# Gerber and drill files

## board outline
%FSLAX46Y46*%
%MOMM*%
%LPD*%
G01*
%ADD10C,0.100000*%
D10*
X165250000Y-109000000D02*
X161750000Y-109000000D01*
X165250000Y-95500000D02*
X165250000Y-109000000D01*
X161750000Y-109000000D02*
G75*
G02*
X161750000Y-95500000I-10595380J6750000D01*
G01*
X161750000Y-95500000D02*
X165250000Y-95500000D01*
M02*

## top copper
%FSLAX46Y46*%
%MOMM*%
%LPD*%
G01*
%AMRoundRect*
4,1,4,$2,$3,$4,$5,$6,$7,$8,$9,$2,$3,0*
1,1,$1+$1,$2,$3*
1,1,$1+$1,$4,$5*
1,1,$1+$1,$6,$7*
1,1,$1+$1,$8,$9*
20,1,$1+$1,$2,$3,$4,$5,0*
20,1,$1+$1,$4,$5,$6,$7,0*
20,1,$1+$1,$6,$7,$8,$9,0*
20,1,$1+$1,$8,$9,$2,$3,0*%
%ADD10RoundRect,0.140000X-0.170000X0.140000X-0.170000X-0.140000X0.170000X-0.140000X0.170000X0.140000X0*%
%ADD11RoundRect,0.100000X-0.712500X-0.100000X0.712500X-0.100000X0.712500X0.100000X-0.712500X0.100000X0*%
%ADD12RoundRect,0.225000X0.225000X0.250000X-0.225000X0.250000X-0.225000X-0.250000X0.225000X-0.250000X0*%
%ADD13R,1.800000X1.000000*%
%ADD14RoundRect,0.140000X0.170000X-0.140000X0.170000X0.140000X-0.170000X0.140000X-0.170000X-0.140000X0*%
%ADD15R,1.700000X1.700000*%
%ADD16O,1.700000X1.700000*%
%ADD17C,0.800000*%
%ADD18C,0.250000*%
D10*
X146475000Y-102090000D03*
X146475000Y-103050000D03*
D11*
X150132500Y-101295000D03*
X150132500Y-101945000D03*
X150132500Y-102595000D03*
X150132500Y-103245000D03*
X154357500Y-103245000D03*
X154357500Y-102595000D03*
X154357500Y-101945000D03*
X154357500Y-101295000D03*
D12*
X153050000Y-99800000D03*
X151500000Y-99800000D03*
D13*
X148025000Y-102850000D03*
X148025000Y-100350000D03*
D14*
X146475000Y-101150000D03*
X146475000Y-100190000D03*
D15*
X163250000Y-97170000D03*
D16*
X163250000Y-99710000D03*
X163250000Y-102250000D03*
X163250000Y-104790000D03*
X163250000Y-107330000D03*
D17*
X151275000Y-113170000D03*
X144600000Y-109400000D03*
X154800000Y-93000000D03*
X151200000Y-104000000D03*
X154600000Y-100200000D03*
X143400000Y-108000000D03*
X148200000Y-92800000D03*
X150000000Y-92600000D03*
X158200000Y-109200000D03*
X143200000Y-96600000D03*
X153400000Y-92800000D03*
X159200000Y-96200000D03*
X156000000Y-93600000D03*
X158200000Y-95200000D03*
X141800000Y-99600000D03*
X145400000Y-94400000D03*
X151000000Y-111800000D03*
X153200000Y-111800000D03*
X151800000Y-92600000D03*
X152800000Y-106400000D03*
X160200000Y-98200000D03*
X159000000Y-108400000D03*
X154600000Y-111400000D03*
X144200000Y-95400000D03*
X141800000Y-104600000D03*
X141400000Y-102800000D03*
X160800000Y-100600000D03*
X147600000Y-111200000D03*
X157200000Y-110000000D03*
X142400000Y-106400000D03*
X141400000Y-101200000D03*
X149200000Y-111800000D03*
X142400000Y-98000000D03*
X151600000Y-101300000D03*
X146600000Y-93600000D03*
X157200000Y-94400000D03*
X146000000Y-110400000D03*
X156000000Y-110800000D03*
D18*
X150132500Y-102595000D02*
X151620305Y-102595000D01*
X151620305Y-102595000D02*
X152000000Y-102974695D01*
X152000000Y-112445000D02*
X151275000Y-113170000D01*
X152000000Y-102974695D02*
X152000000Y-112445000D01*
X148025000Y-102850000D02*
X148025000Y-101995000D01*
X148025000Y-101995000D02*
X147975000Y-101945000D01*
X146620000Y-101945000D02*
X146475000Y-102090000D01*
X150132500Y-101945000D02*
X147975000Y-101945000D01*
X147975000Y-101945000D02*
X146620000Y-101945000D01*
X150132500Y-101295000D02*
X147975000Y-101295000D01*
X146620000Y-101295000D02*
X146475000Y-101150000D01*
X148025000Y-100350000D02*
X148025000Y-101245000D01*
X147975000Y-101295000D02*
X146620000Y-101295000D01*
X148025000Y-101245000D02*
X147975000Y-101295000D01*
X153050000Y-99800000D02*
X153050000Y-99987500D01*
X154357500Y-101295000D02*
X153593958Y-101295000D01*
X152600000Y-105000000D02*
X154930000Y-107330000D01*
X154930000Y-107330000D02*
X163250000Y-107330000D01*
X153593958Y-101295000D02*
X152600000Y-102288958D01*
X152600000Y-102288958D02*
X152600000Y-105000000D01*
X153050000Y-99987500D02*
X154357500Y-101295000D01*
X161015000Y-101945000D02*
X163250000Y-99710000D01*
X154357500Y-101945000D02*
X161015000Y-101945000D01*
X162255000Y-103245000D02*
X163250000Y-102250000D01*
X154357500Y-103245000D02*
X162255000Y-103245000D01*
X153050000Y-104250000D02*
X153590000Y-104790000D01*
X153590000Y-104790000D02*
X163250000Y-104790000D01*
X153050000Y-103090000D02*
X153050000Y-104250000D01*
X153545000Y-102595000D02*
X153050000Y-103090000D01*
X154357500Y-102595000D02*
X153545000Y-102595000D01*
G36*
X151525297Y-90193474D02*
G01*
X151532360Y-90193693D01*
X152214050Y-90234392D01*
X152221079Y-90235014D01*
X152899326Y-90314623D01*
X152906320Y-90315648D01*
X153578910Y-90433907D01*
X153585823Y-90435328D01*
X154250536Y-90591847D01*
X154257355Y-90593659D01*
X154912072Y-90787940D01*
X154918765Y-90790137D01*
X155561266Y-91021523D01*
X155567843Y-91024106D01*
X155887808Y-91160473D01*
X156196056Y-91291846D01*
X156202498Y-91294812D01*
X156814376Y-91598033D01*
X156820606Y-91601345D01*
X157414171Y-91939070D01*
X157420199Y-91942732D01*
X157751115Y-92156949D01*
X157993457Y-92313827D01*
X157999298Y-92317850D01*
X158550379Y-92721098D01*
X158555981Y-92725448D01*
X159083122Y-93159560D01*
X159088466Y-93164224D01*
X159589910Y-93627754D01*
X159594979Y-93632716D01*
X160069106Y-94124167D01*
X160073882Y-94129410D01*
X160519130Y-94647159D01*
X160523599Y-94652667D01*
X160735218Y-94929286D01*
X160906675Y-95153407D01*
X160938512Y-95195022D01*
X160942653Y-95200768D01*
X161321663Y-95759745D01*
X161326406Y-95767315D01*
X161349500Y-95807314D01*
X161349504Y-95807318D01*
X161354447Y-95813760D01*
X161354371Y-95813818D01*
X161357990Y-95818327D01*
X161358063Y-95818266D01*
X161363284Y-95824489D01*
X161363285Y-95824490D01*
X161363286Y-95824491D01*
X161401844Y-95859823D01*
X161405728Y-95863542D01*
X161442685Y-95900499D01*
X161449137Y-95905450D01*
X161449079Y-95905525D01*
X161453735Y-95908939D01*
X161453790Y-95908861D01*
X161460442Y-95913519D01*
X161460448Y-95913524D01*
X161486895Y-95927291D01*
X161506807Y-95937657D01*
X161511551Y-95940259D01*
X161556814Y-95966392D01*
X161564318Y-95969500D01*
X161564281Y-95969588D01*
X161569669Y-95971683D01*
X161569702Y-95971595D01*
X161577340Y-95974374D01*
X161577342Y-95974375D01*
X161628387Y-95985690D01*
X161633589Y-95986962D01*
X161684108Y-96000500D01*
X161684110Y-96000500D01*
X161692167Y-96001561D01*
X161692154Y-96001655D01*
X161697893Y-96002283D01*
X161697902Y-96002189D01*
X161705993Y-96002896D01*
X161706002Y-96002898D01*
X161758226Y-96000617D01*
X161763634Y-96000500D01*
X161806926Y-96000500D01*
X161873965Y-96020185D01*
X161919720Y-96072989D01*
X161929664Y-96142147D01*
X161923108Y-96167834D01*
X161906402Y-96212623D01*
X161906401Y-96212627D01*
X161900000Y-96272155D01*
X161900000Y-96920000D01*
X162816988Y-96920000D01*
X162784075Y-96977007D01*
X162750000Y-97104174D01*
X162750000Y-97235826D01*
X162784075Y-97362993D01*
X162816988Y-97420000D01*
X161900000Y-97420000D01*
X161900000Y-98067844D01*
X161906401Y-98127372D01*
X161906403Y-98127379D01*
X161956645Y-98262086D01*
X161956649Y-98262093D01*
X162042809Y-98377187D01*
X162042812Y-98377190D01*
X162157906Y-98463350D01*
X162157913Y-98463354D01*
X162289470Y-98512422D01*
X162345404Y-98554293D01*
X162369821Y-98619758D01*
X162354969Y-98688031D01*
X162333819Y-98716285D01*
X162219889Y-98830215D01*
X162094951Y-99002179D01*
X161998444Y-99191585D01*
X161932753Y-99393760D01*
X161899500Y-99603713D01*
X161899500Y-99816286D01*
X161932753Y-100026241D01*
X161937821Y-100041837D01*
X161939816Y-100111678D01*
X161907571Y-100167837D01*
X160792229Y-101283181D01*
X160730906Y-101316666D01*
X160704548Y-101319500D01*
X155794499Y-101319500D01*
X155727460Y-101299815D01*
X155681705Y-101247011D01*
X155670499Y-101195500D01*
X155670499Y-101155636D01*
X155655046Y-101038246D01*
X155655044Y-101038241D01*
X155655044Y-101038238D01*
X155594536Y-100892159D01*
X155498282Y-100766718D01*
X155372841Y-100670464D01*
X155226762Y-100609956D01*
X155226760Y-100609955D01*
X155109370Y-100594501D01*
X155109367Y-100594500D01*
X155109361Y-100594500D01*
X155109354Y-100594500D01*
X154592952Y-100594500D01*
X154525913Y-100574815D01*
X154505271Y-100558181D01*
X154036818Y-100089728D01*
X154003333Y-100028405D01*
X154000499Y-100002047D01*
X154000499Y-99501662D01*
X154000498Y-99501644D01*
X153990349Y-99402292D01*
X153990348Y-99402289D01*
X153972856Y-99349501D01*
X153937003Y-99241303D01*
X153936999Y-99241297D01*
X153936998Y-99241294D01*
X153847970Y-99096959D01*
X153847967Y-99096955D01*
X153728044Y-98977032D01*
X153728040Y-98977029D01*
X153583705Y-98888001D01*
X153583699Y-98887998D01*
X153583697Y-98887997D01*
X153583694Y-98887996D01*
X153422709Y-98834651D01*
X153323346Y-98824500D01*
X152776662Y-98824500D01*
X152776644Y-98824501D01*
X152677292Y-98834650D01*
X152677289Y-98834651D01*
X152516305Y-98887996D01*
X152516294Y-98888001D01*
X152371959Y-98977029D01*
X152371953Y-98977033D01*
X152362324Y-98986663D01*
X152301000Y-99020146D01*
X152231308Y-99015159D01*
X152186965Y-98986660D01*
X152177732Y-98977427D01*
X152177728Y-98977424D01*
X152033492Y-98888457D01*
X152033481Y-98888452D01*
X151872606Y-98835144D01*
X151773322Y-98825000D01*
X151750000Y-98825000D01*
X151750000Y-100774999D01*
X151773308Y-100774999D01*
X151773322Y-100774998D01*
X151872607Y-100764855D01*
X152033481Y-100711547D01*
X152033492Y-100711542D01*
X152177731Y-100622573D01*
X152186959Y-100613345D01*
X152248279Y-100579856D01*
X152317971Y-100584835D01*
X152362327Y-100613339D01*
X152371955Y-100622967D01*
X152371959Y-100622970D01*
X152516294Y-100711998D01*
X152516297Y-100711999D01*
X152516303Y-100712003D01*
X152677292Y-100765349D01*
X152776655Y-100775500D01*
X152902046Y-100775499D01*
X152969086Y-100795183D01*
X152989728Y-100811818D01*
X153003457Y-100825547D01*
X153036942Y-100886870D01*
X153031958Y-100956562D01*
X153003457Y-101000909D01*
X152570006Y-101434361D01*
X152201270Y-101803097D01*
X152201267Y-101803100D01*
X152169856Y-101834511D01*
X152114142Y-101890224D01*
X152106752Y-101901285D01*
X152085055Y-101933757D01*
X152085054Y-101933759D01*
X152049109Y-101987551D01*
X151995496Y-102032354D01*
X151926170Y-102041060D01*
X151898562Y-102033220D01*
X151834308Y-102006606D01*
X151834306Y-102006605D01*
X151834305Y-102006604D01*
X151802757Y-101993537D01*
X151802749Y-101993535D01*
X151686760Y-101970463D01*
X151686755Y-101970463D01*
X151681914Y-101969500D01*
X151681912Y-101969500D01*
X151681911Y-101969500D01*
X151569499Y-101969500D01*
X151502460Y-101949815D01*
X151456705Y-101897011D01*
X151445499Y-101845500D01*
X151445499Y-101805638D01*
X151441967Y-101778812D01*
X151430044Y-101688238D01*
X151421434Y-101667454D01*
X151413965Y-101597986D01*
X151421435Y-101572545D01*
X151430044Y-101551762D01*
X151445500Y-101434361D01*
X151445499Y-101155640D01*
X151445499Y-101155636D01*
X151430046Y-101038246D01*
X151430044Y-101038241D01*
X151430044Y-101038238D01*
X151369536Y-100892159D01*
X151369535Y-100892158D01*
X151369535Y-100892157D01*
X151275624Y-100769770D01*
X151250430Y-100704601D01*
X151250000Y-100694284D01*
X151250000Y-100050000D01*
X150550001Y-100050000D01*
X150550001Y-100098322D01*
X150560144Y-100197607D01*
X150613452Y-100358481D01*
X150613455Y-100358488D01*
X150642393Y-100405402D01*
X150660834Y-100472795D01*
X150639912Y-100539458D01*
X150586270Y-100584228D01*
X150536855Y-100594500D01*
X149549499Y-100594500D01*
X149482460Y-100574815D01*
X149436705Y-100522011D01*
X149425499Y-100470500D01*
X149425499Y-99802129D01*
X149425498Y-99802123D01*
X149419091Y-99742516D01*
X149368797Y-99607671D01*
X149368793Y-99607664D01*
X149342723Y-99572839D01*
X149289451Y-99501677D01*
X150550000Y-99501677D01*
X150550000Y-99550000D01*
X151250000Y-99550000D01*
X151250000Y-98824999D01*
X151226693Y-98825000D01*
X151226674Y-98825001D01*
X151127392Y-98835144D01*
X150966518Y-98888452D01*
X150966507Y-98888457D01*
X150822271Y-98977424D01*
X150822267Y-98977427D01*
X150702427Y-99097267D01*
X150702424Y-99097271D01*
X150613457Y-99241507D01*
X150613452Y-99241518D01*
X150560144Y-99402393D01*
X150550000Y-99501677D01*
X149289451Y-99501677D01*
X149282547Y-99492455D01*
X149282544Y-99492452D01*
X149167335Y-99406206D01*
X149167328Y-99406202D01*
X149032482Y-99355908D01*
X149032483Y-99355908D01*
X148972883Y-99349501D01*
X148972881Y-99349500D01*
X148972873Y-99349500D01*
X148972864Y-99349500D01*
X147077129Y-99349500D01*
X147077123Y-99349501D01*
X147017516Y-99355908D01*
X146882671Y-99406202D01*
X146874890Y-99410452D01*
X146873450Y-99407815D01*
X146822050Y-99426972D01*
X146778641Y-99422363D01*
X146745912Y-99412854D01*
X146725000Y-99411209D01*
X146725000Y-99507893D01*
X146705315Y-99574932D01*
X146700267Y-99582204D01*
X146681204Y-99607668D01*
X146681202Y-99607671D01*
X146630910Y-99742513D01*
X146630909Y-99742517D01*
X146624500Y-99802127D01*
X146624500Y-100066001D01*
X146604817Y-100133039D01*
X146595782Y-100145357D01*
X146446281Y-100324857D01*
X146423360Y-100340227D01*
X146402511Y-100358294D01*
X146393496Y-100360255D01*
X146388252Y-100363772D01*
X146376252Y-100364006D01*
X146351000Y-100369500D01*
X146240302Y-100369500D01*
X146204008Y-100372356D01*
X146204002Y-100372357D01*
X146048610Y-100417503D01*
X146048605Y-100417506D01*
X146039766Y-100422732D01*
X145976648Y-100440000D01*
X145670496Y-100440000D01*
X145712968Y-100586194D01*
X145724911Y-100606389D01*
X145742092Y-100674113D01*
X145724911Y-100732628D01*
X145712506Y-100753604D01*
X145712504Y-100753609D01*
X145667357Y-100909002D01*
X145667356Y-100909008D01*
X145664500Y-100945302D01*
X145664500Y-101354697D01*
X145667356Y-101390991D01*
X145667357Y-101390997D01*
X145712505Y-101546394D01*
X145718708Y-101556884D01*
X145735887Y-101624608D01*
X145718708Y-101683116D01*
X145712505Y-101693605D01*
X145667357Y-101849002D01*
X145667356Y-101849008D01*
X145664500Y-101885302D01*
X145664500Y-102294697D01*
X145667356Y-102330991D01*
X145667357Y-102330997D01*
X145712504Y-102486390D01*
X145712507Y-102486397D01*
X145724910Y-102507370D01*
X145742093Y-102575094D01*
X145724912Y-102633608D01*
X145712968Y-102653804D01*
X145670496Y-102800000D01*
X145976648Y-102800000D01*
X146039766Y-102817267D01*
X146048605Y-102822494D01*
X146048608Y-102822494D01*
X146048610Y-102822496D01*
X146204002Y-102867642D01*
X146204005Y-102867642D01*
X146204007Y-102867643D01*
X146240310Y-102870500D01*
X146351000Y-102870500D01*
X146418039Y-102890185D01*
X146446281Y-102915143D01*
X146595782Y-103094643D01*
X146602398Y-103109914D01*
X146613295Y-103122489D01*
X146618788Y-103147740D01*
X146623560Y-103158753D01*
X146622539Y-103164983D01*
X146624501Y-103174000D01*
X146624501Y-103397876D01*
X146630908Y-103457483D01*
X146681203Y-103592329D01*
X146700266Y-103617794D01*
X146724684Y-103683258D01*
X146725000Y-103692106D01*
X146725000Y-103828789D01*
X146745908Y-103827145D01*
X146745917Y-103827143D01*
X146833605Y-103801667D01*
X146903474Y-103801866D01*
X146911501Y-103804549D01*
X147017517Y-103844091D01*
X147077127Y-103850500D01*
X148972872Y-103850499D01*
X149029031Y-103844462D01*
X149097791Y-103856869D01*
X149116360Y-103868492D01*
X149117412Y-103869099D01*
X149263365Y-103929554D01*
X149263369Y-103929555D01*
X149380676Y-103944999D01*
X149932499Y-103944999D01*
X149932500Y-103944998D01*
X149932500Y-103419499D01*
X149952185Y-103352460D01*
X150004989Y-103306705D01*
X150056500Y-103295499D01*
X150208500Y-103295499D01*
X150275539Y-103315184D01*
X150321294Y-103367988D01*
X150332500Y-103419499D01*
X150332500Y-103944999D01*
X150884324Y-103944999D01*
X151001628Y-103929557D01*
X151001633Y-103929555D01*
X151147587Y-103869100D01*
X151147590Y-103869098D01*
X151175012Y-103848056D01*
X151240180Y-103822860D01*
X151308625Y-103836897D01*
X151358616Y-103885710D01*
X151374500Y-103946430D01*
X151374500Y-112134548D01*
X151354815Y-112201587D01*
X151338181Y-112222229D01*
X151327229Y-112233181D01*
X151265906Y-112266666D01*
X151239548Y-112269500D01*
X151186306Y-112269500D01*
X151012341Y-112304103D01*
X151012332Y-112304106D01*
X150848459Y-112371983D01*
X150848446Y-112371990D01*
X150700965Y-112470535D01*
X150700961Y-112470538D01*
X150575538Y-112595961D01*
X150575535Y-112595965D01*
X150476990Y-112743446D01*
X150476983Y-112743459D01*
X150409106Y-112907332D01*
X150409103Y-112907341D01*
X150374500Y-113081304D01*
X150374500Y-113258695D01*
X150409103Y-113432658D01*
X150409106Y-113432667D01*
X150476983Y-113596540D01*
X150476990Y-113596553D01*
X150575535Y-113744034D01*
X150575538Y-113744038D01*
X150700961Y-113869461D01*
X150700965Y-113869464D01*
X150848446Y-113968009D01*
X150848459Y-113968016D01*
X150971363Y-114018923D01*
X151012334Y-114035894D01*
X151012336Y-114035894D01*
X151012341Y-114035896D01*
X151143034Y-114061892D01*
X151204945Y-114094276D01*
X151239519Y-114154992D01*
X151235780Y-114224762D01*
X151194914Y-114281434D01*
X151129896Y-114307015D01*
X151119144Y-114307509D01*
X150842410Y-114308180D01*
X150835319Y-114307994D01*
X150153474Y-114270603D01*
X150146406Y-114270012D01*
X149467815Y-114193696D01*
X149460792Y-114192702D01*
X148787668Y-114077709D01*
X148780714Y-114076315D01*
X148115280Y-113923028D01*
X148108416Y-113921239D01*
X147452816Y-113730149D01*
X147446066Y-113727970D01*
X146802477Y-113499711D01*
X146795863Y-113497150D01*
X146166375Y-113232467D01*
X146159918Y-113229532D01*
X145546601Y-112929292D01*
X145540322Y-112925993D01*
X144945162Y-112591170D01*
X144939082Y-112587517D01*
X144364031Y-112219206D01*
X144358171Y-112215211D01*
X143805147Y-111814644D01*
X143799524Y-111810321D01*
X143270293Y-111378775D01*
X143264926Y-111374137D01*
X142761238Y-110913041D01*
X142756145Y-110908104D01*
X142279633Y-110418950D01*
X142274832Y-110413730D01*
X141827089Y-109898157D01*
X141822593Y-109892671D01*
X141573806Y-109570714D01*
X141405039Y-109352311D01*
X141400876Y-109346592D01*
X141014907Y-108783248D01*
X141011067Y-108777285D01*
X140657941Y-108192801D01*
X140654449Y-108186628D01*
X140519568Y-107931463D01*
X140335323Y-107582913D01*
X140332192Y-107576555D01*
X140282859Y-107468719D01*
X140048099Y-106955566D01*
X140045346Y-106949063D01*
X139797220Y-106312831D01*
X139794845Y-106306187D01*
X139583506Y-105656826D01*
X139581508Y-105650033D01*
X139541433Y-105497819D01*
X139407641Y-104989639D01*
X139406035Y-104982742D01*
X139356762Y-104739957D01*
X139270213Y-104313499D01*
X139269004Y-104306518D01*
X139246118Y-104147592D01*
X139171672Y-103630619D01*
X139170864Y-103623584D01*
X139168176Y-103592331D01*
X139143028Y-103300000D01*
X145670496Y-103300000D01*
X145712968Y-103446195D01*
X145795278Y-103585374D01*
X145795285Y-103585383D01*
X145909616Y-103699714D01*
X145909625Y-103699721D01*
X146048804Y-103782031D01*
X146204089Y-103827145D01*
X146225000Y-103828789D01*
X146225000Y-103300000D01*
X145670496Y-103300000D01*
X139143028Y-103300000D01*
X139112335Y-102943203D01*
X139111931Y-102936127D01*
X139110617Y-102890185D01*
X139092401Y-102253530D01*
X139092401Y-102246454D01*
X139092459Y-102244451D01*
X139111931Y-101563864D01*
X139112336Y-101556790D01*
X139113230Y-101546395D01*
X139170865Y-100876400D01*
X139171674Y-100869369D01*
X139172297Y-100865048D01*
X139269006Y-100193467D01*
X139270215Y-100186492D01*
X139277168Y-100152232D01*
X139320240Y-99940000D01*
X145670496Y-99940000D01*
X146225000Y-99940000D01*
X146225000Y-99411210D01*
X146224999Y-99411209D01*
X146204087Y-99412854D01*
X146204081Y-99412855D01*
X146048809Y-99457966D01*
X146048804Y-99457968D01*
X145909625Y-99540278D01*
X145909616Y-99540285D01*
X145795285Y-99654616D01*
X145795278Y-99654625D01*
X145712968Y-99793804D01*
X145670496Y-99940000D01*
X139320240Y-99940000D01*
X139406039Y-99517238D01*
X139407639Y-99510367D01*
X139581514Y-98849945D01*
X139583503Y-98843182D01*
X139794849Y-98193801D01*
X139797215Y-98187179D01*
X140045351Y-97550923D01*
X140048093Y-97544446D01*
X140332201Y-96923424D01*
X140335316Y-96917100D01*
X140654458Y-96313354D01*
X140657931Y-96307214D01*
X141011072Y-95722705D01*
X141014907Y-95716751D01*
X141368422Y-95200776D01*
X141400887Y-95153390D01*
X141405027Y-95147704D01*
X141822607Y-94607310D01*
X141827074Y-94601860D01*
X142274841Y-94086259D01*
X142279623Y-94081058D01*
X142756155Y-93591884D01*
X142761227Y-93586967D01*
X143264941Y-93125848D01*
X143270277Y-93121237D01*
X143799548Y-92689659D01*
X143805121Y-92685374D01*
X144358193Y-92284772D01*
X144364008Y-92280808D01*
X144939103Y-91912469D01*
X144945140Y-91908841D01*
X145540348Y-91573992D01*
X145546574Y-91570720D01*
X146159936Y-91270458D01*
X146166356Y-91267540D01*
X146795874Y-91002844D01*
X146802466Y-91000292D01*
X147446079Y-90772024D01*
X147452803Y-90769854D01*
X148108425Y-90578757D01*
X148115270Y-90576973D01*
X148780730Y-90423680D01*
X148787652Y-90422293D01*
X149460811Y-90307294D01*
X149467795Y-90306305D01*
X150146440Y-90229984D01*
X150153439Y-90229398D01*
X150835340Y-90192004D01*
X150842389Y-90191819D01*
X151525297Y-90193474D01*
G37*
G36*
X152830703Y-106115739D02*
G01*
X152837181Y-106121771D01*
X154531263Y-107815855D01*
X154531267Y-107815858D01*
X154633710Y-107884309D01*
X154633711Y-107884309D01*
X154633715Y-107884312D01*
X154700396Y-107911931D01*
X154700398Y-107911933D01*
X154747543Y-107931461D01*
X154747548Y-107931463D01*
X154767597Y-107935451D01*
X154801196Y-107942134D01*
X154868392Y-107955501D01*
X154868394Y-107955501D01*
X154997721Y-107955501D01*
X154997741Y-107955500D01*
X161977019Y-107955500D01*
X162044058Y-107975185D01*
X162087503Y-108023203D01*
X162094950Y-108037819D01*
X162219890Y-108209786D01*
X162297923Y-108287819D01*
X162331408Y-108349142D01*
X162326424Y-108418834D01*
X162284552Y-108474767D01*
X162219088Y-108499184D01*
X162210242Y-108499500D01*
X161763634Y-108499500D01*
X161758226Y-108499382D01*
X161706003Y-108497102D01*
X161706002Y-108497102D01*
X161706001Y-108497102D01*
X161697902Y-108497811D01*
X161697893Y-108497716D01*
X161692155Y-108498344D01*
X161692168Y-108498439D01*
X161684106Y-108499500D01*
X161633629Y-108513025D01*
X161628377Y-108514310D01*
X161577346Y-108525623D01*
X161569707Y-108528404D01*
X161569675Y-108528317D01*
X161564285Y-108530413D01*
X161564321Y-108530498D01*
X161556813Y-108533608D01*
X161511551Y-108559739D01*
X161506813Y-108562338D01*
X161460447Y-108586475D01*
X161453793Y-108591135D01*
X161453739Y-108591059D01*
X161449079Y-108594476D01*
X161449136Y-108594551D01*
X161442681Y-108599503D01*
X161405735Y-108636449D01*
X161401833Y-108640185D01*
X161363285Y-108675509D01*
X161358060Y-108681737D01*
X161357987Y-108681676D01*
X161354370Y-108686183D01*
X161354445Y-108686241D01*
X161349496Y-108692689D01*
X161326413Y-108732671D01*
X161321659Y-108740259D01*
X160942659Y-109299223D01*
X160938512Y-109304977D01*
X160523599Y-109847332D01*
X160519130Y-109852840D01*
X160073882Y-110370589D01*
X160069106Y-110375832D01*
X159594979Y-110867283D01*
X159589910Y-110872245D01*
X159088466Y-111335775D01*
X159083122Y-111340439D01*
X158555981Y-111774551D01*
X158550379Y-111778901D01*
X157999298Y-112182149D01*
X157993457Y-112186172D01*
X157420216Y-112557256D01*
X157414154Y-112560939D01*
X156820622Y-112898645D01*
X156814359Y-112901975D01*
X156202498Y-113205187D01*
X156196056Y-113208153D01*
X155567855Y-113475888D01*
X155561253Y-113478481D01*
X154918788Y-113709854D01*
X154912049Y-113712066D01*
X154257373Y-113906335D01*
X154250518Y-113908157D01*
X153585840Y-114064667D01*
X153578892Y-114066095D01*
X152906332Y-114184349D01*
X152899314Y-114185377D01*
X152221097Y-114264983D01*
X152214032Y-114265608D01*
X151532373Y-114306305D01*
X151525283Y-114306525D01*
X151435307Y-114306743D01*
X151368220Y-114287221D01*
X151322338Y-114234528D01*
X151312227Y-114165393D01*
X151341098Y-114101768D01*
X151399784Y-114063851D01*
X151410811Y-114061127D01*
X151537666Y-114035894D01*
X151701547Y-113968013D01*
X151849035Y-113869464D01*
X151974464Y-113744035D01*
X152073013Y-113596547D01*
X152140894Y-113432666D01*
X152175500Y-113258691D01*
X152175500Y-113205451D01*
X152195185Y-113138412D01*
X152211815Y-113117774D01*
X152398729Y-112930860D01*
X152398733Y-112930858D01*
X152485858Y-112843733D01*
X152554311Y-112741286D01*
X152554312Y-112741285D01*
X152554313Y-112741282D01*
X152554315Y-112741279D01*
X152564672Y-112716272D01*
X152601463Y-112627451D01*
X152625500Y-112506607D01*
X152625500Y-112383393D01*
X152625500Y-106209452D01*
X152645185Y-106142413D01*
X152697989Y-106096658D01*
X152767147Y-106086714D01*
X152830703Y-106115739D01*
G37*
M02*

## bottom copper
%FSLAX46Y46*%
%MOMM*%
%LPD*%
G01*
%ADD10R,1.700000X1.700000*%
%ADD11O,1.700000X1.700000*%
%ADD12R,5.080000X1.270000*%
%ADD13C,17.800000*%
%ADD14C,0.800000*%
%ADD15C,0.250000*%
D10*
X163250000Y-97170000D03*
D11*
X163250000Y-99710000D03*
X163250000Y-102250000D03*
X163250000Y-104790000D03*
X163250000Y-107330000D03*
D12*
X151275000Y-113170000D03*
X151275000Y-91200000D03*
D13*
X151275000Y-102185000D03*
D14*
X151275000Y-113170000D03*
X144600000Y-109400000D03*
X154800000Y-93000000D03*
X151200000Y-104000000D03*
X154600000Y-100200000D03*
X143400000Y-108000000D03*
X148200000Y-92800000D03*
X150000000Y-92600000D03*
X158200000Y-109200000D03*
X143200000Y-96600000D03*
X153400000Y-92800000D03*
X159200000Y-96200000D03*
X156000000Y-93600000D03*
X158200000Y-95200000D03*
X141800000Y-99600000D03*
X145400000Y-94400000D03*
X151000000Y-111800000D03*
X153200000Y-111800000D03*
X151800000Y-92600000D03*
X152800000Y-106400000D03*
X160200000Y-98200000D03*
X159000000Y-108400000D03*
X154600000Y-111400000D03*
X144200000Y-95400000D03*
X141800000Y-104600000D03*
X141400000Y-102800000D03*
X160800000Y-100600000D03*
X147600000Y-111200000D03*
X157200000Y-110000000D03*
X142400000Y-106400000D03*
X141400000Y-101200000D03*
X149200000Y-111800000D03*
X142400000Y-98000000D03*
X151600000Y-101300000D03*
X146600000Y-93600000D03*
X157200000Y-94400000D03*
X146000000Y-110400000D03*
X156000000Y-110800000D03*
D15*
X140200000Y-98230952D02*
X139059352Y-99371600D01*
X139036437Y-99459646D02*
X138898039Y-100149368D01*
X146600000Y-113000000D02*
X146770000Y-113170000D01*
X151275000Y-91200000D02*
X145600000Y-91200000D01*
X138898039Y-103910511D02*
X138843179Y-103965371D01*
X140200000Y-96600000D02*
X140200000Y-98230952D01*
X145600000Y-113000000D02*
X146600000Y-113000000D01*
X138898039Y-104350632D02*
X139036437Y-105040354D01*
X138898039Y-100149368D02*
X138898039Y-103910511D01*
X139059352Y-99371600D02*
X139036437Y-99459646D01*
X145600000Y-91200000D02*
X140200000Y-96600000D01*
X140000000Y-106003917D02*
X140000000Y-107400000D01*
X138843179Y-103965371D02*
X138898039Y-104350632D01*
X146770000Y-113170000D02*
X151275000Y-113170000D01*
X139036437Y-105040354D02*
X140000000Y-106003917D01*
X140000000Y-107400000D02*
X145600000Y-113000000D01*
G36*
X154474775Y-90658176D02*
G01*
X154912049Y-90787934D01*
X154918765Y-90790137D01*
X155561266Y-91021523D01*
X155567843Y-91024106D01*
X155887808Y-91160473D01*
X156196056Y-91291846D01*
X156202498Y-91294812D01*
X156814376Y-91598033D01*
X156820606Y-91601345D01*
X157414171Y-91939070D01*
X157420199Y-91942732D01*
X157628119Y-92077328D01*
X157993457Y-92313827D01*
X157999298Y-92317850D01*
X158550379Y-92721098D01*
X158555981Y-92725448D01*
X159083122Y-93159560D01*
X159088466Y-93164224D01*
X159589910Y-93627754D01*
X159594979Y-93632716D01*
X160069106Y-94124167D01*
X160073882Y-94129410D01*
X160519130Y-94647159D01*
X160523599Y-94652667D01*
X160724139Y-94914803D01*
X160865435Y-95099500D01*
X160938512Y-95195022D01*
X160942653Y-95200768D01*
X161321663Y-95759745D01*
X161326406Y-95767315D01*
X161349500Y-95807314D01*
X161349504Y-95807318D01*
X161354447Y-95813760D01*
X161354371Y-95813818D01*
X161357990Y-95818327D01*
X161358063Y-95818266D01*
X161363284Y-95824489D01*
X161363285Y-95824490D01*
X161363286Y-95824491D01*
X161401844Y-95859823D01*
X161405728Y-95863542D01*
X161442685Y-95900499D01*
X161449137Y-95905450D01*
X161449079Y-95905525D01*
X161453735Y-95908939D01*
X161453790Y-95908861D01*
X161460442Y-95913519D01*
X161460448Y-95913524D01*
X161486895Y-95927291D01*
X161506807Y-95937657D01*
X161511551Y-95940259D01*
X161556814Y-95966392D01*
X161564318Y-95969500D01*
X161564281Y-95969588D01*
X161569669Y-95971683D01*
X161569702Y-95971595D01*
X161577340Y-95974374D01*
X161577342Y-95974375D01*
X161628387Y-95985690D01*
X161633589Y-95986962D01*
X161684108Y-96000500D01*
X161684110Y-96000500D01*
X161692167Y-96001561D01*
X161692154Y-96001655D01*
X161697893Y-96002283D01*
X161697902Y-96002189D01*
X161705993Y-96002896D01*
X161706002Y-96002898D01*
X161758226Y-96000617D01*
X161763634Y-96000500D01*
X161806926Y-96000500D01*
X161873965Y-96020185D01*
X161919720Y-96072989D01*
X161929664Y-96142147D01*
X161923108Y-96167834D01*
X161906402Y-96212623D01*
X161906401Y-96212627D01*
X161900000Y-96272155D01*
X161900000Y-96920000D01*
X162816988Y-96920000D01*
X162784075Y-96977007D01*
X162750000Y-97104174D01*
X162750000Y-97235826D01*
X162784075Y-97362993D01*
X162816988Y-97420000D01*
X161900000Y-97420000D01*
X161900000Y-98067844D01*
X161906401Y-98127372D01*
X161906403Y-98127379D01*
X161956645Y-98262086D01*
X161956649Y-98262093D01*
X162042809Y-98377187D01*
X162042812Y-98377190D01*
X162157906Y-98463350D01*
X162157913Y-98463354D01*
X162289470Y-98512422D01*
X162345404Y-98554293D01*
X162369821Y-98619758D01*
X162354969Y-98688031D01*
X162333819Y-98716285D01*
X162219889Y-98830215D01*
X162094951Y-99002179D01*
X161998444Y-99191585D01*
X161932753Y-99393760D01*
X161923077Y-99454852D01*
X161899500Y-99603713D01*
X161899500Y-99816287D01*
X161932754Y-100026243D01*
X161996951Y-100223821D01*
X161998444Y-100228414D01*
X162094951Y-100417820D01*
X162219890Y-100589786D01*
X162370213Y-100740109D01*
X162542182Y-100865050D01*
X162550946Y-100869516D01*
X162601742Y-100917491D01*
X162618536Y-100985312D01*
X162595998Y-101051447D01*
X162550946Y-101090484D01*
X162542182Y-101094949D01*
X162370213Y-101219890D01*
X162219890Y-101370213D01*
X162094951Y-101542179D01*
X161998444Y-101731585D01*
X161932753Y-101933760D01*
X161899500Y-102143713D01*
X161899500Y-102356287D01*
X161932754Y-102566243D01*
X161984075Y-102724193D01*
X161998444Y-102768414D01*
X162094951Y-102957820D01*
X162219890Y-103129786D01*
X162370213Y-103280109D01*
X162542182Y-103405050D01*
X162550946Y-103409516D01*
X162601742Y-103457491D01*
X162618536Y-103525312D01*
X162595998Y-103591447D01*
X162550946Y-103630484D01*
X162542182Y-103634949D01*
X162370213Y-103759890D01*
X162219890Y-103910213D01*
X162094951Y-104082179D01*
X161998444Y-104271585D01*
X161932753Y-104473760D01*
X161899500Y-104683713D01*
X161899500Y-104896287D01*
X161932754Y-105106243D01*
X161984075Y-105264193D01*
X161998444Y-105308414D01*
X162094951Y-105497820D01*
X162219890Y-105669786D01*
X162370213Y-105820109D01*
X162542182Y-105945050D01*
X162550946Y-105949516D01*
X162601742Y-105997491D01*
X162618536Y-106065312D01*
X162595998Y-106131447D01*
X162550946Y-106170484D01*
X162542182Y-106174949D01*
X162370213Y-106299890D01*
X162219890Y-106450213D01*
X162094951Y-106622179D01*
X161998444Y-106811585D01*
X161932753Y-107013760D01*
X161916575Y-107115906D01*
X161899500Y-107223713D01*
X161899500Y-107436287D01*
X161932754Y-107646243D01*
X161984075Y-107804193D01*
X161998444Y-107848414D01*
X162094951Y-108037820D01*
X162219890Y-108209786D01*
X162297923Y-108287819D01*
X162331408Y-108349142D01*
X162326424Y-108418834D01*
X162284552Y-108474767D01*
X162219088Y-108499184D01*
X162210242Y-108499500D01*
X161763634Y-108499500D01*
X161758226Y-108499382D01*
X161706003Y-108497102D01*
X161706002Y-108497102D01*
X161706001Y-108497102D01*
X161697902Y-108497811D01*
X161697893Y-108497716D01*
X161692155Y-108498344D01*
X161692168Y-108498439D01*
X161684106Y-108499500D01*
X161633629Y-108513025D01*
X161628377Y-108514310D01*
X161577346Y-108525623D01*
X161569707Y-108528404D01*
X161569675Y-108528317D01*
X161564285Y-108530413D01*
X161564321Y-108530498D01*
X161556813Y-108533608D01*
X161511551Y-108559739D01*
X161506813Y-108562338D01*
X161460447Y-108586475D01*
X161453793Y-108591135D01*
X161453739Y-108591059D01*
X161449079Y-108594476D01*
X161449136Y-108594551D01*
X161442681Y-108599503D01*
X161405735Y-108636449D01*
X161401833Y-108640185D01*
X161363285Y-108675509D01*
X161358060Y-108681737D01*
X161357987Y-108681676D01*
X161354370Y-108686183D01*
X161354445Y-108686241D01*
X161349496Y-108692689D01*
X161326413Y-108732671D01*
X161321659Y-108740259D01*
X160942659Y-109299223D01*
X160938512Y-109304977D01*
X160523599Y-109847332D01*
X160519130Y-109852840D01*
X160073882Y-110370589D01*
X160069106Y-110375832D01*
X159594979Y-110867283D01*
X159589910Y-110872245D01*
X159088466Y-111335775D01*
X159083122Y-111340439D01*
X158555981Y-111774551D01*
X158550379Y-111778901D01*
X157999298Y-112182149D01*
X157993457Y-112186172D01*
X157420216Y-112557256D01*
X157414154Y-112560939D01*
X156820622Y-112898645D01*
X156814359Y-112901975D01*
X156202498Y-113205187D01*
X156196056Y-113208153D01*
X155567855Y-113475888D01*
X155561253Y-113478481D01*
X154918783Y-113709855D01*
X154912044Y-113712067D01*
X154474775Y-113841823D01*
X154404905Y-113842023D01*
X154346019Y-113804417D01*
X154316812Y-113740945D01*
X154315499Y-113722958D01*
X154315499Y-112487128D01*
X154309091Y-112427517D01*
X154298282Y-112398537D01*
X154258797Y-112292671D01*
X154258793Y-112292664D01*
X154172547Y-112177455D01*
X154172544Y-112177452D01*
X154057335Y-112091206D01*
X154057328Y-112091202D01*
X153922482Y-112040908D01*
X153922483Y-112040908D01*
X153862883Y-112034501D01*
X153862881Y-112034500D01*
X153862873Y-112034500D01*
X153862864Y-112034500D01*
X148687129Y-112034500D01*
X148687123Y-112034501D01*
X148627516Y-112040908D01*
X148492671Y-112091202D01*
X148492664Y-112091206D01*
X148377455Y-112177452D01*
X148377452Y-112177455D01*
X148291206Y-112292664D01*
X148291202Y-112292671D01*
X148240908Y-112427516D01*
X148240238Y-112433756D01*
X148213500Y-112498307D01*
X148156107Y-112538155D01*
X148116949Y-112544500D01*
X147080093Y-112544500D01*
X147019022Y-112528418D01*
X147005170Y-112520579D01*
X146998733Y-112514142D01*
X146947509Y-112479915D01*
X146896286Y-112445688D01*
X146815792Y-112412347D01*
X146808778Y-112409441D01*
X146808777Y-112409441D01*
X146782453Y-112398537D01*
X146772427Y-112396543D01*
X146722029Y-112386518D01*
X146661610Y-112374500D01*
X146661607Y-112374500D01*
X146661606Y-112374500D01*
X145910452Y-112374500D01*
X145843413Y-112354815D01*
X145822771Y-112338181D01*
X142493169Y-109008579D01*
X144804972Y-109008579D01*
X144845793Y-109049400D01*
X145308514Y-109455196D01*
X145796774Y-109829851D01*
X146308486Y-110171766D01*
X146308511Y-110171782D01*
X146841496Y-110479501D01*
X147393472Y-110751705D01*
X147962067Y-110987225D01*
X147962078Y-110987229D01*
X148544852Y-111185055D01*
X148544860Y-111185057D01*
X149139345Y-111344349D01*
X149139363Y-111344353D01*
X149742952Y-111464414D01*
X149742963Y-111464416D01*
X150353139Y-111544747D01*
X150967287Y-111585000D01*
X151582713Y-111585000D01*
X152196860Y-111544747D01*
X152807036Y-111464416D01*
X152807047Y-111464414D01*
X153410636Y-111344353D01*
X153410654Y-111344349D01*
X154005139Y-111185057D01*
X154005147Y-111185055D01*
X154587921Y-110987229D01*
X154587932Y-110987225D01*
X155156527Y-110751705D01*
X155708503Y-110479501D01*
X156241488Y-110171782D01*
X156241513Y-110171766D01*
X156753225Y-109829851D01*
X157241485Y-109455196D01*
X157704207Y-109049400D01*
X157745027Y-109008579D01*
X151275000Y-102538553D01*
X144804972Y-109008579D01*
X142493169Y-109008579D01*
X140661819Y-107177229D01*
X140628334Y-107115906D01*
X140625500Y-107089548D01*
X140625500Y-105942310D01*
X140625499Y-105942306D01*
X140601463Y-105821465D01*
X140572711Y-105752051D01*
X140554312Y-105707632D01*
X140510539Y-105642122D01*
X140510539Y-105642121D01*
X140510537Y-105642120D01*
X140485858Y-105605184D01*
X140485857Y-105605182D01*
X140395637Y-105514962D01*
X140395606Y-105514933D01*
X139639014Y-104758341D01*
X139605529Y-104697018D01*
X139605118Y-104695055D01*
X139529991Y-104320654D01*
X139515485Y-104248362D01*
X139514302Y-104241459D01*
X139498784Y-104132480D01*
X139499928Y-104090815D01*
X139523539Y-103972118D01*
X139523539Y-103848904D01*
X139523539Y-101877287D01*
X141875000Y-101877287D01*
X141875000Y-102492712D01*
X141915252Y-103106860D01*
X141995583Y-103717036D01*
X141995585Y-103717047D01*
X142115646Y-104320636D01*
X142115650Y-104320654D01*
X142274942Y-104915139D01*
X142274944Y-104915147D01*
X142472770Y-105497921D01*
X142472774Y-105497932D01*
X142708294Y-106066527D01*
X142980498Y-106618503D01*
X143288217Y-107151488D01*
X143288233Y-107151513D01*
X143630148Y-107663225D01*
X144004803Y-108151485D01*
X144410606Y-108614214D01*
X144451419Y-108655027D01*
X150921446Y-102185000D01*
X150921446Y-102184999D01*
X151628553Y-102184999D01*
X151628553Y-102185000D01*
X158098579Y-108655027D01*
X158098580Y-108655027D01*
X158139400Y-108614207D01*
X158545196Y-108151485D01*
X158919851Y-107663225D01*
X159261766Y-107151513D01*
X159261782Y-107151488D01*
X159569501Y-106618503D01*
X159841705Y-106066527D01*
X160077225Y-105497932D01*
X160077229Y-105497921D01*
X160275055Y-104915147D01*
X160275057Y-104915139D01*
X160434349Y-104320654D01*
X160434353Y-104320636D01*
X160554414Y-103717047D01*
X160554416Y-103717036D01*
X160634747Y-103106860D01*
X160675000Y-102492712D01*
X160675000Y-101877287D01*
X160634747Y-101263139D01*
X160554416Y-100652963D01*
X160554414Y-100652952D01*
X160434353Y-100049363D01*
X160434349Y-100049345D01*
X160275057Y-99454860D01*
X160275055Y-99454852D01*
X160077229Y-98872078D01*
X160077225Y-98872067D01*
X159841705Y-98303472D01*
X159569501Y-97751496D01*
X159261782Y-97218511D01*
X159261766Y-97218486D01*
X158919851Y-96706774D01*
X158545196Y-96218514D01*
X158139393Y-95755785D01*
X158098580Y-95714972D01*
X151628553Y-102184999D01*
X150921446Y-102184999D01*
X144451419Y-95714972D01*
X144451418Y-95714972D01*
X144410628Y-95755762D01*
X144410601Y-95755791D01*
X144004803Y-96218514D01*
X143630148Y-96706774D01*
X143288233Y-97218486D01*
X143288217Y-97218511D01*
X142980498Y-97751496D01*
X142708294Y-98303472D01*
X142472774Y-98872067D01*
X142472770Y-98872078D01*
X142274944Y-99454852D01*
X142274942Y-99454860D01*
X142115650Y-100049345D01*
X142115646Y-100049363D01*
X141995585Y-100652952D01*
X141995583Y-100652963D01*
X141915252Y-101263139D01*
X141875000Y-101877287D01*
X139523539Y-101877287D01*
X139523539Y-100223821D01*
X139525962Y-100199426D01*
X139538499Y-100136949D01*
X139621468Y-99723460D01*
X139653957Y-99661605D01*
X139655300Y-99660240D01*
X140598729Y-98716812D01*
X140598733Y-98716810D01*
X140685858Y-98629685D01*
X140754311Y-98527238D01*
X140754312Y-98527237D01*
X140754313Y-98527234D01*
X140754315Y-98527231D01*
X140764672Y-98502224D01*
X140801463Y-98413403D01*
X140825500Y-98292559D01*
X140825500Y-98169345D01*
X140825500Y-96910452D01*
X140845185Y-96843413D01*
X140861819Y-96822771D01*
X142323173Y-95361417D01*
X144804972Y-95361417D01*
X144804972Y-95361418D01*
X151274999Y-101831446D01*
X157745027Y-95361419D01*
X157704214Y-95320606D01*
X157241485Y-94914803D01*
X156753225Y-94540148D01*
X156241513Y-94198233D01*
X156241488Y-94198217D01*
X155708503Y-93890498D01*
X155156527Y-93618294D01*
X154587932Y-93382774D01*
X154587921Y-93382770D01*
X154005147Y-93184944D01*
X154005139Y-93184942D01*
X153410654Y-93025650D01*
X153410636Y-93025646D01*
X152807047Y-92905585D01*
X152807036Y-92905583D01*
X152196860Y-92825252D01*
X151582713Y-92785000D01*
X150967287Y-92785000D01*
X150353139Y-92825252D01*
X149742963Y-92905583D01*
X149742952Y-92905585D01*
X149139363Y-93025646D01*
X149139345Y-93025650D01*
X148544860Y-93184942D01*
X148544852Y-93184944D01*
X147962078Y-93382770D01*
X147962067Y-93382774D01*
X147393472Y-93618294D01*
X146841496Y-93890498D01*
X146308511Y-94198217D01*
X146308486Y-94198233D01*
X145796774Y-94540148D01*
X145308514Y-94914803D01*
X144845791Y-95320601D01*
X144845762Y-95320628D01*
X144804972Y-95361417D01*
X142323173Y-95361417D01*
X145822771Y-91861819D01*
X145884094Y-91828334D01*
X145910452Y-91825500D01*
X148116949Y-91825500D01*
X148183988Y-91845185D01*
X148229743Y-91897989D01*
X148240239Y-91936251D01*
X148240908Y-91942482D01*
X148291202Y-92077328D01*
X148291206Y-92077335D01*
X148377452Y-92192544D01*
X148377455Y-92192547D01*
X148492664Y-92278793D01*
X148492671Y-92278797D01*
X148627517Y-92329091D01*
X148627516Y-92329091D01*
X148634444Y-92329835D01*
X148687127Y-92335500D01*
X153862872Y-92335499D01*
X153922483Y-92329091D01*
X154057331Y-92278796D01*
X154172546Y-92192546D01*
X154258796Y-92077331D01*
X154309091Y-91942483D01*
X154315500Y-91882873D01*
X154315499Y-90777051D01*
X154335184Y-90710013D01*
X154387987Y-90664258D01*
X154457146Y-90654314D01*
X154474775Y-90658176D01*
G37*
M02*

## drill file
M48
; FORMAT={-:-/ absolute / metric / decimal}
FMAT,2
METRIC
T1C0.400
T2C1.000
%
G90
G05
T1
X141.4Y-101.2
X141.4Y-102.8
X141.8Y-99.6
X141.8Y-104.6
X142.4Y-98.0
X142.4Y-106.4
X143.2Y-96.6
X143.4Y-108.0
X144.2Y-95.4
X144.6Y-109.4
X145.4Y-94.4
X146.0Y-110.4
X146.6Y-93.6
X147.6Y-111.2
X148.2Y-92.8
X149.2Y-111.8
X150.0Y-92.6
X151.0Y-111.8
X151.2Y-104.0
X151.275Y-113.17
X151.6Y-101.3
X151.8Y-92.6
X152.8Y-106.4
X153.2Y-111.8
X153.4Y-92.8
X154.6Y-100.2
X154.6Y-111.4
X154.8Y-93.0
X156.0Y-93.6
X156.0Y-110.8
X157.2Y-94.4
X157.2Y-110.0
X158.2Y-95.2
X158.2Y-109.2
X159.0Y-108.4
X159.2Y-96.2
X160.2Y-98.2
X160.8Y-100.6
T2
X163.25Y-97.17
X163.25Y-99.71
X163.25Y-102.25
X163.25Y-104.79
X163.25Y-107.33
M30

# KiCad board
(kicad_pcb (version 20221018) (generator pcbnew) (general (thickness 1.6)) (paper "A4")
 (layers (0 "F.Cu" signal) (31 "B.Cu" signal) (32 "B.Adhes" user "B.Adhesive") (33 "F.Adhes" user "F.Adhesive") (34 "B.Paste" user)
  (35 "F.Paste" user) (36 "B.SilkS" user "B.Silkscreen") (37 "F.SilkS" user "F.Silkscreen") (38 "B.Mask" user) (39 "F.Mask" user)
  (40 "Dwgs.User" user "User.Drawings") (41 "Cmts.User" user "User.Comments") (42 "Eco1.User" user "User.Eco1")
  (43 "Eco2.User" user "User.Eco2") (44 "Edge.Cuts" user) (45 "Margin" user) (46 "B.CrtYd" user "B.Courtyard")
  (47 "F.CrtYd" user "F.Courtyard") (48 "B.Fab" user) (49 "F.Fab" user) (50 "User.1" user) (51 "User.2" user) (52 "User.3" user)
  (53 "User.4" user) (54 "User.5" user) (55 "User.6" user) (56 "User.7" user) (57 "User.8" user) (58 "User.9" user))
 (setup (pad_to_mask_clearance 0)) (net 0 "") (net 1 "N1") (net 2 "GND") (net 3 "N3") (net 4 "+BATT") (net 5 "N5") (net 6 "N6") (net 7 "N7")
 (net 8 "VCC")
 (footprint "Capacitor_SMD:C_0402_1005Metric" (layer "F.Cu") (at 146.475 102.57 -90)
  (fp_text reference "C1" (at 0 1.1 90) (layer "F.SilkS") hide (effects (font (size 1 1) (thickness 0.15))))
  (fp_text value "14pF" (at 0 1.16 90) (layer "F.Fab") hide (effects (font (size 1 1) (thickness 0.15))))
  (pad "1" smd roundrect (at -0.48 0 270) (size 0.56 0.62) (layers "F.Cu" "F.Paste" "F.Mask") (roundrect_rratio 0.25) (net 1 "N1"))
  (pad "2" smd roundrect (at 0.48 0 270) (size 0.56 0.62) (layers "F.Cu" "F.Paste" "F.Mask") (roundrect_rratio 0.25) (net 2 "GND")))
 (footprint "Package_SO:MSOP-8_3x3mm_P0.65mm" (layer "F.Cu") (at 152.245 102.27)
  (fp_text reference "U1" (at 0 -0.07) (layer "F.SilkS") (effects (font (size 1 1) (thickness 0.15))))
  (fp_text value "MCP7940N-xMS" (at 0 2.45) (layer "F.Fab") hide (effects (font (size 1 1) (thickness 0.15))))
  (pad "1" smd roundrect (at -2.1125 -0.975) (size 1.625 0.4) (layers "F.Cu" "F.Paste" "F.Mask") (roundrect_rratio 0.25) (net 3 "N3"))
  (pad "2" smd roundrect (at -2.1125 -0.325) (size 1.625 0.4) (layers "F.Cu" "F.Paste" "F.Mask") (roundrect_rratio 0.25) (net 1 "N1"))
  (pad "3" smd roundrect (at -2.1125 0.325) (size 1.625 0.4) (layers "F.Cu" "F.Paste" "F.Mask") (roundrect_rratio 0.25) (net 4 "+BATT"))
  (pad "4" smd roundrect (at -2.1125 0.975) (size 1.625 0.4) (layers "F.Cu" "F.Paste" "F.Mask") (roundrect_rratio 0.25) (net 2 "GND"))
  (pad "5" smd roundrect (at 2.1125 0.975) (size 1.625 0.4) (layers "F.Cu" "F.Paste" "F.Mask") (roundrect_rratio 0.25) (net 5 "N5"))
  (pad "6" smd roundrect (at 2.1125 0.325) (size 1.625 0.4) (layers "F.Cu" "F.Paste" "F.Mask") (roundrect_rratio 0.25) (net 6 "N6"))
  (pad "7" smd roundrect (at 2.1125 -0.325) (size 1.625 0.4) (layers "F.Cu" "F.Paste" "F.Mask") (roundrect_rratio 0.25) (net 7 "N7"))
  (pad "8" smd roundrect (at 2.1125 -0.975) (size 1.625 0.4) (layers "F.Cu" "F.Paste" "F.Mask") (roundrect_rratio 0.25) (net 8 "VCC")))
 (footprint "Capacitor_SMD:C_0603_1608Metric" (layer "F.Cu") (at 152.275 99.8 180)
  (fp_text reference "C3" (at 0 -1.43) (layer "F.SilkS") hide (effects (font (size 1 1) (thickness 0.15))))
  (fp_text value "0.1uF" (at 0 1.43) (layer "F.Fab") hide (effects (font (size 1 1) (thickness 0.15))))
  (pad "1" smd roundrect (at -0.775 0 180) (size 0.9 0.95) (layers "F.Cu" "F.Paste" "F.Mask") (roundrect_rratio 0.25) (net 8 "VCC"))
  (pad "2" smd roundrect (at 0.775 0 180) (size 0.9 0.95) (layers "F.Cu" "F.Paste" "F.Mask") (roundrect_rratio 0.25) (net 2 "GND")))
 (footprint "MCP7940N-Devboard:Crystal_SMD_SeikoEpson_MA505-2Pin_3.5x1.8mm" (layer "F.Cu") (at 148.025 101.6 90)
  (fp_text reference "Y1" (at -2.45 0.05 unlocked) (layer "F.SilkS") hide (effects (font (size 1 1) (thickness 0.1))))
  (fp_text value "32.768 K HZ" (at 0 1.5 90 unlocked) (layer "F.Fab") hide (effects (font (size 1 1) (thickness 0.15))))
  (pad "1" smd rect (at -1.25 0 90) (size 1 1.8) (layers "F.Cu" "F.Paste" "F.Mask") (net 1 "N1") (thermal_bridge_angle 45))
  (pad "2" smd rect (at 1.25 0 90) (size 1 1.8) (layers "F.Cu" "F.Paste" "F.Mask") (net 3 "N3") (thermal_bridge_angle 45)))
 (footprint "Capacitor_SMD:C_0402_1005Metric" (layer "F.Cu") (at 146.475 100.67 90)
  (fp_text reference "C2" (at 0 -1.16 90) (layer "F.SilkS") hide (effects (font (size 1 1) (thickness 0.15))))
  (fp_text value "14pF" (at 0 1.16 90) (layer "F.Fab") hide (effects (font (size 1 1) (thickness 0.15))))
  (pad "1" smd roundrect (at -0.48 0 90) (size 0.56 0.62) (layers "F.Cu" "F.Paste" "F.Mask") (roundrect_rratio 0.25) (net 3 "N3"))
  (pad "2" smd roundrect (at 0.48 0 90) (size 0.56 0.62) (layers "F.Cu" "F.Paste" "F.Mask") (roundrect_rratio 0.25) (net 2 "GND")))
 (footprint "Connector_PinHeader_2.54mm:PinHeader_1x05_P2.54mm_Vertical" (layer "F.Cu") (at 163.25 97.17)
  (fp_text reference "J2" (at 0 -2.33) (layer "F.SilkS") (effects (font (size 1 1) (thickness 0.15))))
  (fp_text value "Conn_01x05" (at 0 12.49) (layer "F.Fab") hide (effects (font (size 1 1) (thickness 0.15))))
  (pad "1" thru_hole rect (at 0 0) (size 1.7 1.7) (drill 1) (layers "*.Cu" "*.Mask") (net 2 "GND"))
  (pad "2" thru_hole oval (at 0 2.54) (size 1.7 1.7) (drill 1) (layers "*.Cu" "*.Mask") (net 7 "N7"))
  (pad "3" thru_hole oval (at 0 5.08) (size 1.7 1.7) (drill 1) (layers "*.Cu" "*.Mask") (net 5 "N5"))
  (pad "4" thru_hole oval (at 0 7.62) (size 1.7 1.7) (drill 1) (layers "*.Cu" "*.Mask") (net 6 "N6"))
  (pad "5" thru_hole oval (at 0 10.16) (size 1.7 1.7) (drill 1) (layers "*.Cu" "*.Mask") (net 8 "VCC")))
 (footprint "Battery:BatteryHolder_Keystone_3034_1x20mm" (layer "B.Cu") (at 151.275 102.185 90)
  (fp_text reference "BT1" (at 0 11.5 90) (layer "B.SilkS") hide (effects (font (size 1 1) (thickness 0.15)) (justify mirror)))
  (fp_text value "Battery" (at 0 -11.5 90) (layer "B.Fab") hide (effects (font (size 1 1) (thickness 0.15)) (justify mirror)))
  (pad "1" smd rect (at -10.985 0 90) (size 1.27 5.08) (layers "B.Cu" "B.Paste" "B.Mask") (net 4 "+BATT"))
  (pad "1" smd rect (at 10.985 0 90) (size 1.27 5.08) (layers "B.Cu" "B.Paste" "B.Mask") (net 4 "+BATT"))
  (pad "2" smd circle (at 0 0 90) (size 17.8 17.8) (layers "B.Cu" "B.Mask") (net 2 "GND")))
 (gr_line (start 165.25 109) (end 161.75 109) (stroke (width 0.1) (type default)) (layer "Edge.Cuts"))
 (gr_line (start 165.25 95.5) (end 165.25 109) (stroke (width 0.1) (type default)) (layer "Edge.Cuts"))
 (gr_arc (start 161.75 109) (mid 138.5918 102.25) (end 161.75 95.5) (stroke (width 0.1) (type default)) (layer "Edge.Cuts"))
 (gr_line (start 161.75 95.5) (end 165.25 95.5) (stroke (width 0.1) (type default)) (layer "Edge.Cuts"))
 (segment (start 150.1325 102.595) (end 151.620305 102.595) (width 0.25) (layer "F.Cu") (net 4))
 (segment (start 151.620305 102.595) (end 152 102.974695) (width 0.25) (layer "F.Cu") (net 4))
 (segment (start 152 112.445) (end 151.275 113.17) (width 0.25) (layer "F.Cu") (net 4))
 (segment (start 152 102.974695) (end 152 112.445) (width 0.25) (layer "F.Cu") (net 4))
 (via (at 151.275 113.17) (size 0.8) (drill 0.4) (layers "F.Cu" "B.Cu") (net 4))
 (segment (start 140.2 98.230952) (end 139.059352 99.3716) (width 0.25) (layer "B.Cu") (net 4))
 (segment (start 139.036437 99.459646) (end 138.898039 100.149368) (width 0.25) (layer "B.Cu") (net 4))
 (segment (start 146.6 113) (end 146.77 113.17) (width 0.25) (layer "B.Cu") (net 4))
 (segment (start 151.275 91.2) (end 145.6 91.2) (width 0.25) (layer "B.Cu") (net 4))
 (segment (start 138.898039 103.910511) (end 138.843179 103.965371) (width 0.25) (layer "B.Cu") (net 4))
 (segment (start 140.2 96.6) (end 140.2 98.230952) (width 0.25) (layer "B.Cu") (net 4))
 (segment (start 145.6 113) (end 146.6 113) (width 0.25) (layer "B.Cu") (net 4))
 (segment (start 138.898039 104.350632) (end 139.036437 105.040354) (width 0.25) (layer "B.Cu") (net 4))
 (segment (start 138.898039 100.149368) (end 138.898039 103.910511) (width 0.25) (layer "B.Cu") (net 4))
 (segment (start 139.059352 99.3716) (end 139.036437 99.459646) (width 0.25) (layer "B.Cu") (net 4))
 (segment (start 145.6 91.2) (end 140.2 96.6) (width 0.25) (layer "B.Cu") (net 4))
 (segment (start 140 106.003917) (end 140 107.4) (width 0.25) (layer "B.Cu") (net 4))
 (segment (start 138.843179 103.965371) (end 138.898039 104.350632) (width 0.25) (layer "B.Cu") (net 4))
 (segment (start 146.77 113.17) (end 151.275 113.17) (width 0.25) (layer "B.Cu") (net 4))
 (segment (start 139.036437 105.040354) (end 140 106.003917) (width 0.25) (layer "B.Cu") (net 4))
 (segment (start 140 107.4) (end 145.6 113) (width 0.25) (layer "B.Cu") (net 4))
 (via (at 144.6 109.4) (size 0.8) (drill 0.4) (layers "F.Cu" "B.Cu") (free) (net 2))
 (via (at 154.8 93) (size 0.8) (drill 0.4) (layers "F.Cu" "B.Cu") (free) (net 2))
 (via (at 151.2 104) (size 0.8) (drill 0.4) (layers "F.Cu" "B.Cu") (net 2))
 (via (at 154.6 100.2) (size 0.8) (drill 0.4) (layers "F.Cu" "B.Cu") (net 2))
 (via (at 143.4 108) (size 0.8) (drill 0.4) (layers "F.Cu" "B.Cu") (free) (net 2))
 (via (at 148.2 92.8) (size 0.8) (drill 0.4) (layers "F.Cu" "B.Cu") (free) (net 2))
 (via (at 150 92.6) (size 0.8) (drill 0.4) (layers "F.Cu" "B.Cu") (free) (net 2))
 (via (at 158.2 109.2) (size 0.8) (drill 0.4) (layers "F.Cu" "B.Cu") (free) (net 2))
 (via (at 143.2 96.6) (size 0.8) (drill 0.4) (layers "F.Cu" "B.Cu") (free) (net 2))
 (via (at 153.4 92.8) (size 0.8) (drill 0.4) (layers "F.Cu" "B.Cu") (free) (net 2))
 (via (at 159.2 96.2) (size 0.8) (drill 0.4) (layers "F.Cu" "B.Cu") (free) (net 2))
 (via (at 156 93.6) (size 0.8) (drill 0.4) (layers "F.Cu" "B.Cu") (free) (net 2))
 (via (at 158.2 95.2) (size 0.8) (drill 0.4) (layers "F.Cu" "B.Cu") (free) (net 2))
 (via (at 141.8 99.6) (size 0.8) (drill 0.4) (layers "F.Cu" "B.Cu") (free) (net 2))
 (via (at 145.4 94.4) (size 0.8) (drill 0.4) (layers "F.Cu" "B.Cu") (free) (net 2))
 (via (at 151 111.8) (size 0.8) (drill 0.4) (layers "F.Cu" "B.Cu") (free) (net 2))
 (via (at 153.2 111.8) (size 0.8) (drill 0.4) (layers "F.Cu" "B.Cu") (free) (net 2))
 (via (at 151.8 92.6) (size 0.8) (drill 0.4) (layers "F.Cu" "B.Cu") (free) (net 2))
 (via (at 152.8 106.4) (size 0.8) (drill 0.4) (layers "F.Cu" "B.Cu") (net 2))
 (via (at 160.2 98.2) (size 0.8) (drill 0.4) (layers "F.Cu" "B.Cu") (free) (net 2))
 (via (at 159 108.4) (size 0.8) (drill 0.4) (layers "F.Cu" "B.Cu") (free) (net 2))
 (via (at 154.6 111.4) (size 0.8) (drill 0.4) (layers "F.Cu" "B.Cu") (free) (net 2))
 (via (at 144.2 95.4) (size 0.8) (drill 0.4) (layers "F.Cu" "B.Cu") (free) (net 2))
 (via (at 141.8 104.6) (size 0.8) (drill 0.4) (layers "F.Cu" "B.Cu") (free) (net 2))
 (via (at 141.4 102.8) (size 0.8) (drill 0.4) (layers "F.Cu" "B.Cu") (free) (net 2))
 (via (at 160.8 100.6) (size 0.8) (drill 0.4) (layers "F.Cu" "B.Cu") (free) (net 2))
 (via (at 147.6 111.2) (size 0.8) (drill 0.4) (layers "F.Cu" "B.Cu") (free) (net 2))
 (via (at 157.2 110) (size 0.8) (drill 0.4) (layers "F.Cu" "B.Cu") (free) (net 2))
 (via (at 142.4 106.4) (size 0.8) (drill 0.4) (layers "F.Cu" "B.Cu") (free) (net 2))
 (via (at 141.4 101.2) (size 0.8) (drill 0.4) (layers "F.Cu" "B.Cu") (free) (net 2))
 (via (at 149.2 111.8) (size 0.8) (drill 0.4) (layers "F.Cu" "B.Cu") (free) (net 2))
 (via (at 142.4 98) (size 0.8) (drill 0.4) (layers "F.Cu" "B.Cu") (free) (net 2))
 (via (at 151.6 101.3) (size 0.8) (drill 0.4) (layers "F.Cu" "B.Cu") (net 2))
 (via (at 146.6 93.6) (size 0.8) (drill 0.4) (layers "F.Cu" "B.Cu") (free) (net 2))
 (via (at 157.2 94.4) (size 0.8) (drill 0.4) (layers "F.Cu" "B.Cu") (free) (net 2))
 (via (at 146 110.4) (size 0.8) (drill 0.4) (layers "F.Cu" "B.Cu") (free) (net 2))
 (via (at 156 110.8) (size 0.8) (drill 0.4) (layers "F.Cu" "B.Cu") (free) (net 2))
 (segment (start 148.025 102.85) (end 148.025 101.995) (width 0.25) (layer "F.Cu") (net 1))
 (segment (start 148.025 101.995) (end 147.975 101.945) (width 0.25) (layer "F.Cu") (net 1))
 (segment (start 146.62 101.945) (end 146.475 102.09) (width 0.25) (layer "F.Cu") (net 1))
 (segment (start 150.1325 101.945) (end 147.975 101.945) (width 0.25) (layer "F.Cu") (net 1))
 (segment (start 147.975 101.945) (end 146.62 101.945) (width 0.25) (layer "F.Cu") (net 1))
 (segment (start 150.1325 101.295) (end 147.975 101.295) (width 0.25) (layer "F.Cu") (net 3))
 (segment (start 146.62 101.295) (end 146.475 101.15) (width 0.25) (layer "F.Cu") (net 3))
 (segment (start 148.025 100.35) (end 148.025 101.245) (width 0.25) (layer "F.Cu") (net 3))
 (segment (start 147.975 101.295) (end 146.62 101.295) (width 0.25) (layer "F.Cu") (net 3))
 (segment (start 148.025 101.245) (end 147.975 101.295) (width 0.25) (layer "F.Cu") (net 3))
 (segment (start 153.05 99.8) (end 153.05 99.9875) (width 0.25) (layer "F.Cu") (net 8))
 (segment (start 154.3575 101.295) (end 153.593958 101.295) (width 0.25) (layer "F.Cu") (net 8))
 (segment (start 152.6 105) (end 154.93 107.33) (width 0.25) (layer "F.Cu") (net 8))
 (segment (start 154.93 107.33) (end 163.25 107.33) (width 0.25) (layer "F.Cu") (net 8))
 (segment (start 153.593958 101.295) (end 152.6 102.288958) (width 0.25) (layer "F.Cu") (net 8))
 (segment (start 152.6 102.288958) (end 152.6 105) (width 0.25) (layer "F.Cu") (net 8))
 (segment (start 153.05 99.9875) (end 154.3575 101.295) (width 0.25) (layer "F.Cu") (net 8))
 (segment (start 161.015 101.945) (end 163.25 99.71) (width 0.25) (layer "F.Cu") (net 7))
 (segment (start 154.3575 101.945) (end 161.015 101.945) (width 0.25) (layer "F.Cu") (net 7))
 (segment (start 162.255 103.245) (end 163.25 102.25) (width 0.25) (layer "F.Cu") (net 5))
 (segment (start 154.3575 103.245) (end 162.255 103.245) (width 0.25) (layer "F.Cu") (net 5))
 (segment (start 153.05 104.25) (end 153.59 104.79) (width 0.25) (layer "F.Cu") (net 6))
 (segment (start 153.59 104.79) (end 163.25 104.79) (width 0.25) (layer "F.Cu") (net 6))
 (segment (start 153.05 103.09) (end 153.05 104.25) (width 0.25) (layer "F.Cu") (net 6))
 (segment (start 153.545 102.595) (end 153.05 103.09) (width 0.25) (layer "F.Cu") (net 6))
 (segment (start 154.3575 102.595) (end 153.545 102.595) (width 0.25) (layer "F.Cu") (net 6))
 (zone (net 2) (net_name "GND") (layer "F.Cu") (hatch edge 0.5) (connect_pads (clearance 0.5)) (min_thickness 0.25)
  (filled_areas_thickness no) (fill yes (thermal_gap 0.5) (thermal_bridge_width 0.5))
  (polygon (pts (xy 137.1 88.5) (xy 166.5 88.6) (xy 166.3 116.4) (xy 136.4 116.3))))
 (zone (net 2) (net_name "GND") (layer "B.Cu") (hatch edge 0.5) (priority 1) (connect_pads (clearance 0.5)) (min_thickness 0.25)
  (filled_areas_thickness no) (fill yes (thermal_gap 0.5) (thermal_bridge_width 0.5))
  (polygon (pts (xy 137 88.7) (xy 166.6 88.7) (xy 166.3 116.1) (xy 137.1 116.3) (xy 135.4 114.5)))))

